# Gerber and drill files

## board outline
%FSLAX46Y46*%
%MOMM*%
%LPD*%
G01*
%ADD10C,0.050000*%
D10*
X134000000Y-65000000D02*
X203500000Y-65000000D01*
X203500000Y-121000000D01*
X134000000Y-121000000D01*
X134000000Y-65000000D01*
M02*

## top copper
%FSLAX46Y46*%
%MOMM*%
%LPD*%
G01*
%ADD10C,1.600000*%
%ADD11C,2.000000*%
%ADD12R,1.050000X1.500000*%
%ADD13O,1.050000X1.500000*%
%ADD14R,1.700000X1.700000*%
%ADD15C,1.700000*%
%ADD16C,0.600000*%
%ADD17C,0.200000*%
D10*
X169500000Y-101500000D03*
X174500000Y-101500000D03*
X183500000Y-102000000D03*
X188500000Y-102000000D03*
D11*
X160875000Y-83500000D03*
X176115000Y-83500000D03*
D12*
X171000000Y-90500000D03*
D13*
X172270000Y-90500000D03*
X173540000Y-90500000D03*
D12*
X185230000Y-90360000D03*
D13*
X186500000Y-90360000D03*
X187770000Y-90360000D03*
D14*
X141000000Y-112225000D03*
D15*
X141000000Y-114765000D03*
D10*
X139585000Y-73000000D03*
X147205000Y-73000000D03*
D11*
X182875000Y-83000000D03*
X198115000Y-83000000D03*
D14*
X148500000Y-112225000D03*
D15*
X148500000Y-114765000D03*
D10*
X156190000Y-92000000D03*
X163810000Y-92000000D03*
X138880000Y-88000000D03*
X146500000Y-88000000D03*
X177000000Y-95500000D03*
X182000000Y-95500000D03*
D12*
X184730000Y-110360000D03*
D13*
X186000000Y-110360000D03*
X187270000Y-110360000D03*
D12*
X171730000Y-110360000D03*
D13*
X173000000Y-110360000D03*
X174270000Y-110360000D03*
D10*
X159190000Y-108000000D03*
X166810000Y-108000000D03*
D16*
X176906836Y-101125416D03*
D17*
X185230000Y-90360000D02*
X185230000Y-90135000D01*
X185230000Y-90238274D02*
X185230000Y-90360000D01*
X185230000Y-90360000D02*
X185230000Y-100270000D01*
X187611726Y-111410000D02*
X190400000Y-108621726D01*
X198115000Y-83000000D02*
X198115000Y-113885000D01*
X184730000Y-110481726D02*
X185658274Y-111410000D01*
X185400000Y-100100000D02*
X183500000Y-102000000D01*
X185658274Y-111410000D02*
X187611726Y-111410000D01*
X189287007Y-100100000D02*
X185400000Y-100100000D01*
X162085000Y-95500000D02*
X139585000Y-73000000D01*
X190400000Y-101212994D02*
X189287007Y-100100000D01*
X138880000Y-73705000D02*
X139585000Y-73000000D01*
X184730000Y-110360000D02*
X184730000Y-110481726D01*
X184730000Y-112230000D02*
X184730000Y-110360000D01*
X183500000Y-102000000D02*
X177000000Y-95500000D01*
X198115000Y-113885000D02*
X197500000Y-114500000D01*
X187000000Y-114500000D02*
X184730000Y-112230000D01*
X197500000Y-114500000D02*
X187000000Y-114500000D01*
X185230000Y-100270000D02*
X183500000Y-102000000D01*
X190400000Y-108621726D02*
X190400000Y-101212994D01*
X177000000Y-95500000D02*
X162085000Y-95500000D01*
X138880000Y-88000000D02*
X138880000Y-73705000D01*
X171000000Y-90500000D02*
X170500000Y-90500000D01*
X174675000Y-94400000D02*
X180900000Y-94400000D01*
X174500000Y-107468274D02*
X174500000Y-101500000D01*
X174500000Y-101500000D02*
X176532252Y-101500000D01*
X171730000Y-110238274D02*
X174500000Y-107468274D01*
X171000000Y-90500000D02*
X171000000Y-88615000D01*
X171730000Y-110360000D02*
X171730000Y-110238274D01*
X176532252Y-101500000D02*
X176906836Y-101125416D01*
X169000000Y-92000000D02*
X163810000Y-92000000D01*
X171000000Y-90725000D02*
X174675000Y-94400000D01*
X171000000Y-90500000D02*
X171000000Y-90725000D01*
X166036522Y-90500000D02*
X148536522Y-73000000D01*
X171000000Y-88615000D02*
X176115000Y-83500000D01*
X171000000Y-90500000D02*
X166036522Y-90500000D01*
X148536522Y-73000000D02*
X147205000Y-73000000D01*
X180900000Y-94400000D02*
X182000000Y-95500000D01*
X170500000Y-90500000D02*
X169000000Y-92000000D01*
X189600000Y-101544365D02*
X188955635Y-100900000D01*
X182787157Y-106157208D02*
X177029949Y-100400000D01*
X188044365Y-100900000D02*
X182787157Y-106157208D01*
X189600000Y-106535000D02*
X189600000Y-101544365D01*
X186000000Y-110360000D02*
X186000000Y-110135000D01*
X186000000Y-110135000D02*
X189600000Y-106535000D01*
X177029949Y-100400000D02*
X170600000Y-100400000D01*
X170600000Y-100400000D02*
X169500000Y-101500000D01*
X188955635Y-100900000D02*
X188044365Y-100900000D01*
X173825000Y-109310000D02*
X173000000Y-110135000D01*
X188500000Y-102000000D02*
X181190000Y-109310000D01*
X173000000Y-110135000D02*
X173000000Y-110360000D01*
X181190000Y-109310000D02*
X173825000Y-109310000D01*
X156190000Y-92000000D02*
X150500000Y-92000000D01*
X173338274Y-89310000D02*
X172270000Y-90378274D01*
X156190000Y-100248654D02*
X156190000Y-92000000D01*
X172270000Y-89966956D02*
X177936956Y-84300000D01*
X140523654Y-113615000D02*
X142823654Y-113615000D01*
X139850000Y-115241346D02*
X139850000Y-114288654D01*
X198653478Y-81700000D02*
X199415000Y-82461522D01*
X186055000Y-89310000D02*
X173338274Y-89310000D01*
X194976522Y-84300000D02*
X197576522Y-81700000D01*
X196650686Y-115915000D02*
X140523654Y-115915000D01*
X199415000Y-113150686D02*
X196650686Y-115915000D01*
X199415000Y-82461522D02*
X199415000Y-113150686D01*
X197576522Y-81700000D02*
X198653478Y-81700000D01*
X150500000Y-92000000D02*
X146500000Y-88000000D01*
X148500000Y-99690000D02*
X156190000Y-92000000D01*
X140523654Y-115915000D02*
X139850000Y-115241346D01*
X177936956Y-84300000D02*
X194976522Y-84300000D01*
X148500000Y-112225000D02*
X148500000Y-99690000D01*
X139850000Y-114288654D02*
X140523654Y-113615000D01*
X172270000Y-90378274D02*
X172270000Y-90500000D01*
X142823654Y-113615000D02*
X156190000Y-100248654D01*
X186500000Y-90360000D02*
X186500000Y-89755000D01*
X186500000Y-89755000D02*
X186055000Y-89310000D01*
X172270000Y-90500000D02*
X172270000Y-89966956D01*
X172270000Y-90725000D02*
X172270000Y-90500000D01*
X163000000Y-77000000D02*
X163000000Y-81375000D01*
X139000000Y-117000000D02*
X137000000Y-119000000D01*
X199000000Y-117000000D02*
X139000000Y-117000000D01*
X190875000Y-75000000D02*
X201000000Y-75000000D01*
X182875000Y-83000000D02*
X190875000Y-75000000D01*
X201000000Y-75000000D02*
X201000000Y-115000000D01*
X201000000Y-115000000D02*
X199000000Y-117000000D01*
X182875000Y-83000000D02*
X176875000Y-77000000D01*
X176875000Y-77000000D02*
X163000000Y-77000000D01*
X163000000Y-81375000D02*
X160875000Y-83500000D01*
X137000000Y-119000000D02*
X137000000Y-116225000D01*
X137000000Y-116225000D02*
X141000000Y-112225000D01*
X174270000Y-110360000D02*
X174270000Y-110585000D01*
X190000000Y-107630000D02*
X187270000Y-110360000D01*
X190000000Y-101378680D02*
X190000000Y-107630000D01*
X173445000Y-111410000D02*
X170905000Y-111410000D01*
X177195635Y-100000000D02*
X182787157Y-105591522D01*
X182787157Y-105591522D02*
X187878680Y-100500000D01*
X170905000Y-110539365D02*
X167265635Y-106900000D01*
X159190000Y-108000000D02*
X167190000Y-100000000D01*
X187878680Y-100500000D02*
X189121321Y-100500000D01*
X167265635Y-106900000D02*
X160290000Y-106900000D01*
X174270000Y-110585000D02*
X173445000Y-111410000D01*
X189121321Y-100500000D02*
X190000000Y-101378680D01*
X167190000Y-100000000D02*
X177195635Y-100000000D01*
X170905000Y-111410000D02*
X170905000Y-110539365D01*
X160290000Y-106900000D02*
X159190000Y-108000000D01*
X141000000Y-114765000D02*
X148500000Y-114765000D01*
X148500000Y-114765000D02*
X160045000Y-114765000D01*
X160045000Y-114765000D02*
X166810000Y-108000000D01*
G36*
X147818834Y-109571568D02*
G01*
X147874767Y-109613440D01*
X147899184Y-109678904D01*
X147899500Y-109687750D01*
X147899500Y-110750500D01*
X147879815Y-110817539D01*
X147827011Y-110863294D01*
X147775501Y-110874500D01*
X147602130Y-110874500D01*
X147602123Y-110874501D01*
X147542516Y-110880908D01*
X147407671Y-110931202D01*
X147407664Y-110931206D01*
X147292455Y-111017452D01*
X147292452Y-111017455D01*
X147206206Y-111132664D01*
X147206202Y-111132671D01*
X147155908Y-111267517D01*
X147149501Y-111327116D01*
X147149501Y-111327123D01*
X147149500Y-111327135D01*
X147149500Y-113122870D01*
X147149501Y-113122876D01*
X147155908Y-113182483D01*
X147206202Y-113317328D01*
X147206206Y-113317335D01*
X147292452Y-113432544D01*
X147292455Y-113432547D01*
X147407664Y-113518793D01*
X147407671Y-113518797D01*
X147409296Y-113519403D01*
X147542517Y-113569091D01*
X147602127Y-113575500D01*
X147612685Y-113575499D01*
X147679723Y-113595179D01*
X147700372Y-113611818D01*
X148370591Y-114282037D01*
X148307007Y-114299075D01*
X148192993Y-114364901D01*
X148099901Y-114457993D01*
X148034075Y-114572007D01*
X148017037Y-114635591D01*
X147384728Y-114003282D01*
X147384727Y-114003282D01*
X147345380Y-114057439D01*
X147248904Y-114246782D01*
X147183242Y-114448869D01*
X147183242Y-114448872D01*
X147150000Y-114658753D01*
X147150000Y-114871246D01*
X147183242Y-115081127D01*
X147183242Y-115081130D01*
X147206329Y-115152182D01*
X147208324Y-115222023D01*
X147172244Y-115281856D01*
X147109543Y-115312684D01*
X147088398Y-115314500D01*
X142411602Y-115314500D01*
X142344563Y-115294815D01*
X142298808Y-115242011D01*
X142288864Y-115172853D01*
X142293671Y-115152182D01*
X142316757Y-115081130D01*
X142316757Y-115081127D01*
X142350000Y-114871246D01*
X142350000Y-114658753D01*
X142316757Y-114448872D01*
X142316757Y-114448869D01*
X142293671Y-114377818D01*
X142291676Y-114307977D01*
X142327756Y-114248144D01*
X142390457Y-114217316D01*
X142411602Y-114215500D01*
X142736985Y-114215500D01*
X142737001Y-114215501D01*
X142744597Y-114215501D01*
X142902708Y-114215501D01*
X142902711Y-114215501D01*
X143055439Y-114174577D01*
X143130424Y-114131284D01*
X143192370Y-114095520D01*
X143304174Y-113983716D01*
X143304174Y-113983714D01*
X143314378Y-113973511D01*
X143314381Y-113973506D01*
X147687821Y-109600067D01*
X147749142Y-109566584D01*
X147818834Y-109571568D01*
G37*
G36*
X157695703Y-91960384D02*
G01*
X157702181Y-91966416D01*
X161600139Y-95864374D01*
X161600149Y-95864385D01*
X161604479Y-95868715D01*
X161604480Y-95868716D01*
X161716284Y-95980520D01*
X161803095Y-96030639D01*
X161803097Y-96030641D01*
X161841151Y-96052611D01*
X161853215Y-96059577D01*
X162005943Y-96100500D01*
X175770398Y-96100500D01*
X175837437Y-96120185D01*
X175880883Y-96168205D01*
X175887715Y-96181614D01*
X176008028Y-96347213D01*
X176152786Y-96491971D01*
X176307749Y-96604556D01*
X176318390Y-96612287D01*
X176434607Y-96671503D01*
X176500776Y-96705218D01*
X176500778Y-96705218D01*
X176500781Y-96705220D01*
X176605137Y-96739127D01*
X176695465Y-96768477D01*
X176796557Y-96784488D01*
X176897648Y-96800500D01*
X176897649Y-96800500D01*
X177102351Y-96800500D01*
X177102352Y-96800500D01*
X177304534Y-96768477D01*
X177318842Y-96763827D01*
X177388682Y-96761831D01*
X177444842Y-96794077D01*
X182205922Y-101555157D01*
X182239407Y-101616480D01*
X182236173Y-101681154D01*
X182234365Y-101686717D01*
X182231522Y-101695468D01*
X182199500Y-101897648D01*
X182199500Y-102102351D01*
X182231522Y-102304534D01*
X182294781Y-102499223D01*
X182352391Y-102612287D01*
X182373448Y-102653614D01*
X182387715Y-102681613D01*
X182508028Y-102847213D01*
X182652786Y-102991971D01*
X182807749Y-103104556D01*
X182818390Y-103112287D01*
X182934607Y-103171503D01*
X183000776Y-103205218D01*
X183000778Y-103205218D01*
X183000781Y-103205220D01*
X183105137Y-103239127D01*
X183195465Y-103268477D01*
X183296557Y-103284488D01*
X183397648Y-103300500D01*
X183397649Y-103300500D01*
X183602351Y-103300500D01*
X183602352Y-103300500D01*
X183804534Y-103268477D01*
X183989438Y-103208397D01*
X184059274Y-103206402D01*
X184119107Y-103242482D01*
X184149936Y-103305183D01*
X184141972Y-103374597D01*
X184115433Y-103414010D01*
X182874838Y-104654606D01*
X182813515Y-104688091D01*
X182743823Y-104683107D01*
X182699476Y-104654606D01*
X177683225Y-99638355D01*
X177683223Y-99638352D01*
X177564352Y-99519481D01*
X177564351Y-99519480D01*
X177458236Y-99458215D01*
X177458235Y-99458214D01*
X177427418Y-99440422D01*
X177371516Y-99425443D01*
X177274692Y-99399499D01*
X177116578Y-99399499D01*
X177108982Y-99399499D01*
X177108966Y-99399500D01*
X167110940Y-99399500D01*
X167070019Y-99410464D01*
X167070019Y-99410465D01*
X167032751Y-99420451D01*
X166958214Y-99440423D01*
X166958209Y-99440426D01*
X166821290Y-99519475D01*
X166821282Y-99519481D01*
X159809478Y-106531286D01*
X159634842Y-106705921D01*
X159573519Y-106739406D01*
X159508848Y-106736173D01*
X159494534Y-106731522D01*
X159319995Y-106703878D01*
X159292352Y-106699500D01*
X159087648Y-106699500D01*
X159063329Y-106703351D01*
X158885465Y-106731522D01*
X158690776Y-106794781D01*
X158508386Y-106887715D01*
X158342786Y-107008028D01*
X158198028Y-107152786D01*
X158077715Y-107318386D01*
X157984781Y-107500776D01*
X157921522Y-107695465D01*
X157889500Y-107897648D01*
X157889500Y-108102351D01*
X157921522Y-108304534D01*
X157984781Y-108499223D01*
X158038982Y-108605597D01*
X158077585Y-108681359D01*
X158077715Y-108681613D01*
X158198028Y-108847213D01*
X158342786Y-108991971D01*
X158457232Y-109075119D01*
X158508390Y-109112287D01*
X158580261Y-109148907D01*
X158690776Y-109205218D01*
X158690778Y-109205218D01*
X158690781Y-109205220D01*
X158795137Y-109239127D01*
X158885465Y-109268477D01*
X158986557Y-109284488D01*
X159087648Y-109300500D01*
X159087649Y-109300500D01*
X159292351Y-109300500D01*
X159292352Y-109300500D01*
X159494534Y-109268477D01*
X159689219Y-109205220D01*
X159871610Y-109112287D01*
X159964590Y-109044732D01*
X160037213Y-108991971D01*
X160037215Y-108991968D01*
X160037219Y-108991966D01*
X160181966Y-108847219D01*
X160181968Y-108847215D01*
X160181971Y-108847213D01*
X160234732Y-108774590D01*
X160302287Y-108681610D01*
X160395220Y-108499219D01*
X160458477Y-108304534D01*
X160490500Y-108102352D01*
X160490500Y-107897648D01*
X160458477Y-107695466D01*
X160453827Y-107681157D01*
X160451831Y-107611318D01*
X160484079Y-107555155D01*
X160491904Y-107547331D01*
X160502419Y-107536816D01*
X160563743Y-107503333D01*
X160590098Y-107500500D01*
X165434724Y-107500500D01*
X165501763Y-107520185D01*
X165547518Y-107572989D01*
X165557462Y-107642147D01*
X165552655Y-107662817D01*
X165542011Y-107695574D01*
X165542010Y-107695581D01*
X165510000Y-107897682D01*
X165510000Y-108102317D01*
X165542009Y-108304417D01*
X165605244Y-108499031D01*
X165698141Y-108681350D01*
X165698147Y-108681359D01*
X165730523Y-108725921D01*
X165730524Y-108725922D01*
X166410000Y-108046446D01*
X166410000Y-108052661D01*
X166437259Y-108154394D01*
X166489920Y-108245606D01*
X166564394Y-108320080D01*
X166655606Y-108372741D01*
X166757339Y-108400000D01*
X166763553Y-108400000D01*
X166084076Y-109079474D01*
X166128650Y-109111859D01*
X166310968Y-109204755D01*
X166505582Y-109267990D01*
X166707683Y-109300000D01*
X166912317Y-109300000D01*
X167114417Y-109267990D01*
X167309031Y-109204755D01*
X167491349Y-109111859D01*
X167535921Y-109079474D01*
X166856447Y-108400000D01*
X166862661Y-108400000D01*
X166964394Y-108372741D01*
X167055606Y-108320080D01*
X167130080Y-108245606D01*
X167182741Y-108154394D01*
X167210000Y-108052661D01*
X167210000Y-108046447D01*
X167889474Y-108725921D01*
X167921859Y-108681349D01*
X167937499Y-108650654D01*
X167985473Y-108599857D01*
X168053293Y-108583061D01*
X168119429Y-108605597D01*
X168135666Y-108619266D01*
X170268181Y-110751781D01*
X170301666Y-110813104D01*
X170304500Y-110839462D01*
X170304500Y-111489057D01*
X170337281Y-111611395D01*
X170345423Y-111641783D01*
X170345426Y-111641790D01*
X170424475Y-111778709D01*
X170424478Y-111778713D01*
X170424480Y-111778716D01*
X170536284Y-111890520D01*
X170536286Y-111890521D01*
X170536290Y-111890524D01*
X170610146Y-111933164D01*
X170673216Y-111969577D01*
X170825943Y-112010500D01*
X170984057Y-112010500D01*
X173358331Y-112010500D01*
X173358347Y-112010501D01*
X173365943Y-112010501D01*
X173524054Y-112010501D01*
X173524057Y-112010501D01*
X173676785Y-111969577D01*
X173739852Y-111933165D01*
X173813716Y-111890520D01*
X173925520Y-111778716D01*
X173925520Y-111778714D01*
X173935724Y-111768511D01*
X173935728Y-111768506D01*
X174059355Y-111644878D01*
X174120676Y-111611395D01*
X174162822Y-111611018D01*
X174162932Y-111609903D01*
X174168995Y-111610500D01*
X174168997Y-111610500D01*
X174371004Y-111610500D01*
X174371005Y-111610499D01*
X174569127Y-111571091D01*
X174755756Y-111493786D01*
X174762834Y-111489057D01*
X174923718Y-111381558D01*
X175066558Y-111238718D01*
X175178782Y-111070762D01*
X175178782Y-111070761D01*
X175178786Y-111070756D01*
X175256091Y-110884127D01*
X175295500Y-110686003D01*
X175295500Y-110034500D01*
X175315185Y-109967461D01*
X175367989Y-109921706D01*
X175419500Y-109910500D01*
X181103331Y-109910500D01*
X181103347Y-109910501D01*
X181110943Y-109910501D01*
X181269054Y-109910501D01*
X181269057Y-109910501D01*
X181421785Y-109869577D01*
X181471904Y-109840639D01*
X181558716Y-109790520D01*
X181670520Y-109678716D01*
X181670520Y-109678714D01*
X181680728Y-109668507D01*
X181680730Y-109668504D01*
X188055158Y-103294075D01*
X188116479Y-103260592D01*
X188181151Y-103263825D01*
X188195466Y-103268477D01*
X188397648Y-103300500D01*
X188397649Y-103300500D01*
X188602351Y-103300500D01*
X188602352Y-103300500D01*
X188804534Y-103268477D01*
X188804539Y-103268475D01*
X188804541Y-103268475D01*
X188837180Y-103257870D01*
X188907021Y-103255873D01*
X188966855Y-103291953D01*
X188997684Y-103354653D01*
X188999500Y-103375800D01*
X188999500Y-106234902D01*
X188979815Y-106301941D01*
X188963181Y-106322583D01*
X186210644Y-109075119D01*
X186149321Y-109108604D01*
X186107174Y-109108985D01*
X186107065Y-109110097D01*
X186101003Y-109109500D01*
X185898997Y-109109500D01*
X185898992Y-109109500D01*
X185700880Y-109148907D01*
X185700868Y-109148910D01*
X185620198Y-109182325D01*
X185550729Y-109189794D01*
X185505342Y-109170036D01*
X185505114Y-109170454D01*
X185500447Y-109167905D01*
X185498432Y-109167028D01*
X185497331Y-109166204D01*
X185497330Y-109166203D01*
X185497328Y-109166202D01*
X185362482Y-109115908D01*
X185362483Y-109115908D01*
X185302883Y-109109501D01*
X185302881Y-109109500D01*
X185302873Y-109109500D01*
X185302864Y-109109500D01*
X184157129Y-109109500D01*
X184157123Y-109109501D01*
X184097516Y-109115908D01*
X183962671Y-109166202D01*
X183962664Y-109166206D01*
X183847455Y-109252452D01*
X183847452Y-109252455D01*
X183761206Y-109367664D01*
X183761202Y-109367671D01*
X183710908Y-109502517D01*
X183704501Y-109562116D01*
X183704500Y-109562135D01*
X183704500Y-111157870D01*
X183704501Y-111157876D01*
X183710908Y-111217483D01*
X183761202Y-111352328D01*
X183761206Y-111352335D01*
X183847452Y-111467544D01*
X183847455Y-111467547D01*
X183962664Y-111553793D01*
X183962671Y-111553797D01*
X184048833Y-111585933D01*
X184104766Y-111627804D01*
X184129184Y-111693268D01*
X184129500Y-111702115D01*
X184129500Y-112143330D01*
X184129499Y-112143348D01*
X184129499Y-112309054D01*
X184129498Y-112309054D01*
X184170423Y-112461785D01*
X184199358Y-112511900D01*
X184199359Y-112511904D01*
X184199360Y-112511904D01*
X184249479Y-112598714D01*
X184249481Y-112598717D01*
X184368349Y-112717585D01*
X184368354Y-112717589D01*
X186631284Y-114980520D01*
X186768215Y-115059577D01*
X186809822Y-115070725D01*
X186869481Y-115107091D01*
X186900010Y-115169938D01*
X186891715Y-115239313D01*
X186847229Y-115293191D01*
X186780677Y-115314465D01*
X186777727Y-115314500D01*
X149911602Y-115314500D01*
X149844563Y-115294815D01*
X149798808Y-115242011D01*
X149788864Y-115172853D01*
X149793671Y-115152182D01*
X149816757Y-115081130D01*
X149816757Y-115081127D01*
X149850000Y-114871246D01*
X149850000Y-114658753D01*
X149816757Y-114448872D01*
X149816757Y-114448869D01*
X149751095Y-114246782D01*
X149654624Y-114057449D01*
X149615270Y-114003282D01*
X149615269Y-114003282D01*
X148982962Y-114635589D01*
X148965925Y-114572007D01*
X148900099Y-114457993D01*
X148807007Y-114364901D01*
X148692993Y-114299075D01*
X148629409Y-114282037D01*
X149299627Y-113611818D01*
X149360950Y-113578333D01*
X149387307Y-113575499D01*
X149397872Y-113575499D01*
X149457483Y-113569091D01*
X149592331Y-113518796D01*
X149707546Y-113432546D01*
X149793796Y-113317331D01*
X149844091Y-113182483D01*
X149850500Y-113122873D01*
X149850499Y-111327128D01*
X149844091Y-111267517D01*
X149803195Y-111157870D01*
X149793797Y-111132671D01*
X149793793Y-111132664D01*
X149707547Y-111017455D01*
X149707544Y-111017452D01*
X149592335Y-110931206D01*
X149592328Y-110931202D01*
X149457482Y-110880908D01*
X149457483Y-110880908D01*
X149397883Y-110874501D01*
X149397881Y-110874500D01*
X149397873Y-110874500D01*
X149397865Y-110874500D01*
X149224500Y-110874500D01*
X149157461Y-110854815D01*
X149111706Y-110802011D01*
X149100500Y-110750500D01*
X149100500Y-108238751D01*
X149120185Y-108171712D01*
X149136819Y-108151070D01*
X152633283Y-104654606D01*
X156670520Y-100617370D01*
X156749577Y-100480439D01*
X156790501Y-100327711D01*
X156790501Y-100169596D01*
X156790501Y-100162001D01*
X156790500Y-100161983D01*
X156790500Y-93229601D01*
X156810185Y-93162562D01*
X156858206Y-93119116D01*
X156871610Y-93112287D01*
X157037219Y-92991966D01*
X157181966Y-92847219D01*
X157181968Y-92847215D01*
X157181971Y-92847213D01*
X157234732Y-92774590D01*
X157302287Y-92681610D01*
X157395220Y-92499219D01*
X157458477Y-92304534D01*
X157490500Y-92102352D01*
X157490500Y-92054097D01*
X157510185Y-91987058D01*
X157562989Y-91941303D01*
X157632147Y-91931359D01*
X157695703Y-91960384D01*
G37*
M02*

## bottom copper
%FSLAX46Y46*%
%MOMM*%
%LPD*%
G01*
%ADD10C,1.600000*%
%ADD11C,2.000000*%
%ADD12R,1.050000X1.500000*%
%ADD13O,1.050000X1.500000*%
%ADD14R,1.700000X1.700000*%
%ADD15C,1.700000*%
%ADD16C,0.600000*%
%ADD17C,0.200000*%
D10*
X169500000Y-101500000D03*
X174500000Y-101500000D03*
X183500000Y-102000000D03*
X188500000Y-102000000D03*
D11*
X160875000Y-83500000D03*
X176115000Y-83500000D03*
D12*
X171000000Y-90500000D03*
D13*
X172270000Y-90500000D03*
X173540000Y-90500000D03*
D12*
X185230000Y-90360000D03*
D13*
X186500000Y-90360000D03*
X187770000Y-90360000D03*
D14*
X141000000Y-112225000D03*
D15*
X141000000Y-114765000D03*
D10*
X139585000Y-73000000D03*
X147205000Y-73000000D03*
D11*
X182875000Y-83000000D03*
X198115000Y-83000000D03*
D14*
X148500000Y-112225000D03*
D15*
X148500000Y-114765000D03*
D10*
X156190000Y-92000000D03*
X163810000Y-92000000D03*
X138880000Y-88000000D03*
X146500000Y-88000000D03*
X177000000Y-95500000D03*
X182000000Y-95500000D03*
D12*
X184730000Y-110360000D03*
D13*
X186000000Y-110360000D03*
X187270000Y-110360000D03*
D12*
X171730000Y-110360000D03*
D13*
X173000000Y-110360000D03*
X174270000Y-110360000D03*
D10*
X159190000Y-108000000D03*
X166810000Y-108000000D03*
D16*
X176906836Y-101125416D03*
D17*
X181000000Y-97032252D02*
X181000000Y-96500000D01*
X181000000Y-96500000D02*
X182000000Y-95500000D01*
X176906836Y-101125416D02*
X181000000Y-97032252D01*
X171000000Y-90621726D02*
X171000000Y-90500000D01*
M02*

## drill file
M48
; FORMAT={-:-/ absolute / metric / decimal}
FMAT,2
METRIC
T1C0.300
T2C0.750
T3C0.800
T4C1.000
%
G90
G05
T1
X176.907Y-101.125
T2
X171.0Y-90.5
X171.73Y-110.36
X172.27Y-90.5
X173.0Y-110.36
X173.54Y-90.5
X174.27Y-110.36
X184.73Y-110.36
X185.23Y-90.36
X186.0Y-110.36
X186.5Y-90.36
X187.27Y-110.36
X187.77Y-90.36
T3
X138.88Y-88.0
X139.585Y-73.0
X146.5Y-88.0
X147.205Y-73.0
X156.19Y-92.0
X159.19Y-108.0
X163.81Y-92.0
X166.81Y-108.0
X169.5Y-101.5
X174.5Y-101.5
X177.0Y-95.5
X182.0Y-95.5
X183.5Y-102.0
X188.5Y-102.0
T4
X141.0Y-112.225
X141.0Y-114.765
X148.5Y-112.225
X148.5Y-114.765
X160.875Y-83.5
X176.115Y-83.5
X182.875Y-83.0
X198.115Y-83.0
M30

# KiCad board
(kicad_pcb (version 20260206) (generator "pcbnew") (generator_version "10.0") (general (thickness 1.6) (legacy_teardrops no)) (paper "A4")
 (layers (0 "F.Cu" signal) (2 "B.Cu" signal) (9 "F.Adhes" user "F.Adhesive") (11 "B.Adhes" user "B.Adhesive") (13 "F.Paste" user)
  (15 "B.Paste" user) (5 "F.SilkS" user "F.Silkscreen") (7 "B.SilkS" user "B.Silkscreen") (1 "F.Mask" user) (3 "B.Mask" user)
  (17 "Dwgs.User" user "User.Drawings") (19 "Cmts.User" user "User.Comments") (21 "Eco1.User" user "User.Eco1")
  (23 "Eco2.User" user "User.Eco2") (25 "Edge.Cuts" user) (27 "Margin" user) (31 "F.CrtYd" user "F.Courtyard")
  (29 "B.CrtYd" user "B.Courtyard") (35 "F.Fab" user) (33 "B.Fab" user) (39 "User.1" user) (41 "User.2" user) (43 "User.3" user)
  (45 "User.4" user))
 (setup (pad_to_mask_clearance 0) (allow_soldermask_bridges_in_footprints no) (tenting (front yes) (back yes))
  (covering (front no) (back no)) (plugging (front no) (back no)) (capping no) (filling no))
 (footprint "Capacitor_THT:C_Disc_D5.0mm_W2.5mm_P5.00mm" (layer "F.Cu") (at 169.5 101.5)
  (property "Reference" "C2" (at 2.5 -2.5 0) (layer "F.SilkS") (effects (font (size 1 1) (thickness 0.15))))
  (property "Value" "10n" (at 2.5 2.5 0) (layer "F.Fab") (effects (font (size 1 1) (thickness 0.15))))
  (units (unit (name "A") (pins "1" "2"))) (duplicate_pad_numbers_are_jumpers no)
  (pad "1" thru_hole circle (at 0 0) (size 1.6 1.6) (drill 0.8) (layers "*.Cu" "*.Mask") (remove_unused_layers no) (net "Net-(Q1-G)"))
  (pad "2" thru_hole circle (at 5 0) (size 1.6 1.6) (drill 0.8) (layers "*.Cu" "*.Mask") (remove_unused_layers no) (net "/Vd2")))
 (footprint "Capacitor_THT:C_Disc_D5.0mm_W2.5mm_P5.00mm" (layer "F.Cu") (at 183.5 102)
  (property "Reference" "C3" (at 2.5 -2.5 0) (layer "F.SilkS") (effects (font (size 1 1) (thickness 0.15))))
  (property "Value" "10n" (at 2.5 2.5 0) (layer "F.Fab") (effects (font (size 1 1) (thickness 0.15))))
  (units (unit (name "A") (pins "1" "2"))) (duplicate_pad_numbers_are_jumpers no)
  (pad "1" thru_hole circle (at 0 0) (size 1.6 1.6) (drill 0.8) (layers "*.Cu" "*.Mask") (remove_unused_layers no) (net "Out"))
  (pad "2" thru_hole circle (at 5 0) (size 1.6 1.6) (drill 0.8) (layers "*.Cu" "*.Mask") (remove_unused_layers no) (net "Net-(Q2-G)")))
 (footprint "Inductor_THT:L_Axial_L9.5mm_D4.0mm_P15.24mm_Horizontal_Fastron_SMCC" (layer "F.Cu") (at 160.875 83.5)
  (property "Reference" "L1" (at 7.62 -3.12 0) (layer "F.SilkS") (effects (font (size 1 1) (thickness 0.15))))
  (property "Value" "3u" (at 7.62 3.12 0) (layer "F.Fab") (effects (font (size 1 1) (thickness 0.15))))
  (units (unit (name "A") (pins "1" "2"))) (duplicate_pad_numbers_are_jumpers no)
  (pad "1" thru_hole circle (at 0 0) (size 2 2) (drill 1) (layers "*.Cu" "*.Mask") (remove_unused_layers no) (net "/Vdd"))
  (pad "2" thru_hole circle (at 15.24 0) (size 2 2) (drill 1) (layers "*.Cu" "*.Mask") (remove_unused_layers no) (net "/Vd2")))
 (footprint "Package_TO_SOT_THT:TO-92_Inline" (layer "F.Cu") (at 171 90.5)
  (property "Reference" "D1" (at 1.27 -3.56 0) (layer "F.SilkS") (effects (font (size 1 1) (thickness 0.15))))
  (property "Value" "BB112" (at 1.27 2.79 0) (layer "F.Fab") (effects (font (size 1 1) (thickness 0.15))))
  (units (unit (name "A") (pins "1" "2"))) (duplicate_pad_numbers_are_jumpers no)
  (pad "1" thru_hole rect (at 0 0) (size 1.05 1.5) (drill 0.75) (layers "*.Cu" "*.Mask") (remove_unused_layers no) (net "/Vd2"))
  (pad "2" thru_hole oval (at 1.27 0) (size 1.05 1.5) (drill 0.75) (layers "*.Cu" "*.Mask") (remove_unused_layers no) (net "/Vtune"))
  (pad "3" thru_hole oval (at 2.54 0) (size 1.05 1.5) (drill 0.75) (layers "*.Cu" "*.Mask") (remove_unused_layers no)))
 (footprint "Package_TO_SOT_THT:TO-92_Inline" (layer "F.Cu") (at 185.23 90.36)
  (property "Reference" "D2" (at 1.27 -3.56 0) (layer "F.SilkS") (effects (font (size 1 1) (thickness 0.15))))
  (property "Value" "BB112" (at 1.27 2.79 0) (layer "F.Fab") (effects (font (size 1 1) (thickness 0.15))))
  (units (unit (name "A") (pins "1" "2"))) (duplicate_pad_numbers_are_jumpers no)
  (pad "1" thru_hole rect (at 0 0) (size 1.05 1.5) (drill 0.75) (layers "*.Cu" "*.Mask") (remove_unused_layers no) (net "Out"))
  (pad "2" thru_hole oval (at 1.27 0) (size 1.05 1.5) (drill 0.75) (layers "*.Cu" "*.Mask") (remove_unused_layers no) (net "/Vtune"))
  (pad "3" thru_hole oval (at 2.54 0) (size 1.05 1.5) (drill 0.75) (layers "*.Cu" "*.Mask") (remove_unused_layers no)))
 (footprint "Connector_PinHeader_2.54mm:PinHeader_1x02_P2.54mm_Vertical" (layer "F.Cu") (at 141 112.225)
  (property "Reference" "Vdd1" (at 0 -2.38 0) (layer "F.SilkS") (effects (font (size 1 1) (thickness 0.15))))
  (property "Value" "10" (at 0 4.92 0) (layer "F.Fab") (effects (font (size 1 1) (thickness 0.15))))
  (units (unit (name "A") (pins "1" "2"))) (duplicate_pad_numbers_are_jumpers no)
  (pad "1" thru_hole rect (at 0 0) (size 1.7 1.7) (drill 1) (layers "*.Cu" "*.Mask") (remove_unused_layers no) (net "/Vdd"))
  (pad "2" thru_hole circle (at 0 2.54) (size 1.7 1.7) (drill 1) (layers "*.Cu" "*.Mask") (remove_unused_layers no) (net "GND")))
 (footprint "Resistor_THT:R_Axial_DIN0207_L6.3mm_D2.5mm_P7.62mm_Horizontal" (layer "F.Cu") (at 139.585 73)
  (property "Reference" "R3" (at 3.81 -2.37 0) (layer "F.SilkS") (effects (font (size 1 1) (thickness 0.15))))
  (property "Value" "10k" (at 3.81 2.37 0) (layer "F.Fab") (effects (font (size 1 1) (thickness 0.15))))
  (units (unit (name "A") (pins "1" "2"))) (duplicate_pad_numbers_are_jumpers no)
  (pad "1" thru_hole circle (at 0 0) (size 1.6 1.6) (drill 0.8) (layers "*.Cu" "*.Mask") (remove_unused_layers no) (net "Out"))
  (pad "2" thru_hole circle (at 7.62 0) (size 1.6 1.6) (drill 0.8) (layers "*.Cu" "*.Mask") (remove_unused_layers no) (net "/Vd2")))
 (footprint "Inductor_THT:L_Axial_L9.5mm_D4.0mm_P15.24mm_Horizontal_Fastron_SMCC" (layer "F.Cu") (at 182.875 83)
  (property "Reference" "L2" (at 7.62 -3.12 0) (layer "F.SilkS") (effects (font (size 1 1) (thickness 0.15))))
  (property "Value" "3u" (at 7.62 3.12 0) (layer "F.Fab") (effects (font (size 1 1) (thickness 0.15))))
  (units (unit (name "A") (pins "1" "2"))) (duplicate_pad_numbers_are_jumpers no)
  (pad "1" thru_hole circle (at 0 0) (size 2 2) (drill 1) (layers "*.Cu" "*.Mask") (remove_unused_layers no) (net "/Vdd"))
  (pad "2" thru_hole circle (at 15.24 0) (size 2 2) (drill 1) (layers "*.Cu" "*.Mask") (remove_unused_layers no) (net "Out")))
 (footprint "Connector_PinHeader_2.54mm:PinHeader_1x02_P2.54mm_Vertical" (layer "F.Cu") (at 148.5 112.225)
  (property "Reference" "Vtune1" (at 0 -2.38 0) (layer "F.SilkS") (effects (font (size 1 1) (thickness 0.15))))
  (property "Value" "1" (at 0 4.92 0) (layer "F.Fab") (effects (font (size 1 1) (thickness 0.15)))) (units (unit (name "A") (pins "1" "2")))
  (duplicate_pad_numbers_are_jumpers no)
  (pad "1" thru_hole rect (at 0 0) (size 1.7 1.7) (drill 1) (layers "*.Cu" "*.Mask") (remove_unused_layers no) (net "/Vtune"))
  (pad "2" thru_hole circle (at 0 2.54) (size 1.7 1.7) (drill 1) (layers "*.Cu" "*.Mask") (remove_unused_layers no) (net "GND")))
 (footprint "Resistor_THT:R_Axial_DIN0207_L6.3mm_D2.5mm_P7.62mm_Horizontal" (layer "F.Cu") (at 156.19 92)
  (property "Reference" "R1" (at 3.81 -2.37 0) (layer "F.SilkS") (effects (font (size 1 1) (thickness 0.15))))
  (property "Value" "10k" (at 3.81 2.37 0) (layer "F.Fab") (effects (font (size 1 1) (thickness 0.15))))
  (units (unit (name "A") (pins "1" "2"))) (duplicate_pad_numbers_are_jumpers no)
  (pad "1" thru_hole circle (at 0 0) (size 1.6 1.6) (drill 0.8) (layers "*.Cu" "*.Mask") (remove_unused_layers no) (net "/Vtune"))
  (pad "2" thru_hole circle (at 7.62 0) (size 1.6 1.6) (drill 0.8) (layers "*.Cu" "*.Mask") (remove_unused_layers no) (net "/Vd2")))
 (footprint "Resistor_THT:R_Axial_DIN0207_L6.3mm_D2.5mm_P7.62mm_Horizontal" (layer "F.Cu") (at 138.88 88)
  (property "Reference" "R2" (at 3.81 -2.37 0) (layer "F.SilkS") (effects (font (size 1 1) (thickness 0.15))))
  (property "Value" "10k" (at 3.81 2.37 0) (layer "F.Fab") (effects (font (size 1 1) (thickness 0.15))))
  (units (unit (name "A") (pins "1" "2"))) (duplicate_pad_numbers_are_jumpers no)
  (pad "1" thru_hole circle (at 0 0) (size 1.6 1.6) (drill 0.8) (layers "*.Cu" "*.Mask") (remove_unused_layers no) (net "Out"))
  (pad "2" thru_hole circle (at 7.62 0) (size 1.6 1.6) (drill 0.8) (layers "*.Cu" "*.Mask") (remove_unused_layers no) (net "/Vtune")))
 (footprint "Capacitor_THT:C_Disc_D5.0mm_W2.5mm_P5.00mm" (layer "F.Cu") (at 177 95.5)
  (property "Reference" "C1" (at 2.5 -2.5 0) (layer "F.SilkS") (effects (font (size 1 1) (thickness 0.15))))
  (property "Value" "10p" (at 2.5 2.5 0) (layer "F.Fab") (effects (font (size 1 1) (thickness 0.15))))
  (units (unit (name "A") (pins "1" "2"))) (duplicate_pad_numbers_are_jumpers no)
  (pad "1" thru_hole circle (at 0 0) (size 1.6 1.6) (drill 0.8) (layers "*.Cu" "*.Mask") (remove_unused_layers no) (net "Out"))
  (pad "2" thru_hole circle (at 5 0) (size 1.6 1.6) (drill 0.8) (layers "*.Cu" "*.Mask") (remove_unused_layers no) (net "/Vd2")))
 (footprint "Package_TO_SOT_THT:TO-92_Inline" (layer "F.Cu") (at 184.73 110.36)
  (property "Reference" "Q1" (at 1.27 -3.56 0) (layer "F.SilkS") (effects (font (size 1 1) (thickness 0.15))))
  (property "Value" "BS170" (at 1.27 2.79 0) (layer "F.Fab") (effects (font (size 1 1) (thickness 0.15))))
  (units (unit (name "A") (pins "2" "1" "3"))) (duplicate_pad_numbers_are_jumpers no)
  (pad "1" thru_hole rect (at 0 0) (size 1.05 1.5) (drill 0.75) (layers "*.Cu" "*.Mask") (remove_unused_layers no) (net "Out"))
  (pad "2" thru_hole oval (at 1.27 0) (size 1.05 1.5) (drill 0.75) (layers "*.Cu" "*.Mask") (remove_unused_layers no) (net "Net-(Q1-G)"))
  (pad "3" thru_hole oval (at 2.54 0) (size 1.05 1.5) (drill 0.75) (layers "*.Cu" "*.Mask") (remove_unused_layers no) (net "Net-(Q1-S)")))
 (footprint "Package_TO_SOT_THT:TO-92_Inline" (layer "F.Cu") (at 171.73 110.36)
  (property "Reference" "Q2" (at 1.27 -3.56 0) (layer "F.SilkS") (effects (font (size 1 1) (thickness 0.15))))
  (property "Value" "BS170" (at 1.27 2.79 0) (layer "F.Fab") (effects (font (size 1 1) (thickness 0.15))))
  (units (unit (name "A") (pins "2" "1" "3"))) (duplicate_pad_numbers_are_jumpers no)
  (pad "1" thru_hole rect (at 0 0) (size 1.05 1.5) (drill 0.75) (layers "*.Cu" "*.Mask") (remove_unused_layers no) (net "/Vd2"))
  (pad "2" thru_hole oval (at 1.27 0) (size 1.05 1.5) (drill 0.75) (layers "*.Cu" "*.Mask") (remove_unused_layers no) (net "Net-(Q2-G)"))
  (pad "3" thru_hole oval (at 2.54 0) (size 1.05 1.5) (drill 0.75) (layers "*.Cu" "*.Mask") (remove_unused_layers no) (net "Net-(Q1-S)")))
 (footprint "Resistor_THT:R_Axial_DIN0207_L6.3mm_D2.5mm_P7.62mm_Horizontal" (layer "F.Cu") (at 159.19 108)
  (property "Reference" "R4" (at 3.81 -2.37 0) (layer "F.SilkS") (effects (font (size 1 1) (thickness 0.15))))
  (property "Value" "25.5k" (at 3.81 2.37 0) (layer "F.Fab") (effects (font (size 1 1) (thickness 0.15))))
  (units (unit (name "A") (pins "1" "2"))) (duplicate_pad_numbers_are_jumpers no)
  (pad "1" thru_hole circle (at 0 0) (size 1.6 1.6) (drill 0.8) (layers "*.Cu" "*.Mask") (remove_unused_layers no) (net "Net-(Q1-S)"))
  (pad "2" thru_hole circle (at 7.62 0) (size 1.6 1.6) (drill 0.8) (layers "*.Cu" "*.Mask") (remove_unused_layers no) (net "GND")))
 (gr_rect (start 134 65) (end 203.5 121) (stroke (width 0.05) (type default)) (fill no) (layer "Edge.Cuts"))
 (segment (start 185.23 90.36) (end 185.23 90.135) (width 0.2) (layer "F.Cu") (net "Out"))
 (segment (start 185.23 90.238274) (end 185.23 90.36) (width 0.2) (layer "F.Cu") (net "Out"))
 (segment (start 185.23 90.36) (end 185.23 100.27) (width 0.2) (layer "F.Cu") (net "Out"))
 (segment (start 187.611726 111.41) (end 190.4 108.621726) (width 0.2) (layer "F.Cu") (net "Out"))
 (segment (start 198.115 83) (end 198.115 113.885) (width 0.2) (layer "F.Cu") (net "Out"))
 (segment (start 184.73 110.481726) (end 185.658274 111.41) (width 0.2) (layer "F.Cu") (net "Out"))
 (segment (start 185.4 100.1) (end 183.5 102) (width 0.2) (layer "F.Cu") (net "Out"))
 (segment (start 185.658274 111.41) (end 187.611726 111.41) (width 0.2) (layer "F.Cu") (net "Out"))
 (segment (start 189.287007 100.1) (end 185.4 100.1) (width 0.2) (layer "F.Cu") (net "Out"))
 (segment (start 162.085 95.5) (end 139.585 73) (width 0.2) (layer "F.Cu") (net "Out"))
 (segment (start 190.4 101.212994) (end 189.287007 100.1) (width 0.2) (layer "F.Cu") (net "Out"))
 (segment (start 138.88 73.705) (end 139.585 73) (width 0.2) (layer "F.Cu") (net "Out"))
 (segment (start 184.73 110.36) (end 184.73 110.481726) (width 0.2) (layer "F.Cu") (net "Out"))
 (segment (start 184.73 112.23) (end 184.73 110.36) (width 0.2) (layer "F.Cu") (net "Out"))
 (segment (start 183.5 102) (end 177 95.5) (width 0.2) (layer "F.Cu") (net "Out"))
 (segment (start 198.115 113.885) (end 197.5 114.5) (width 0.2) (layer "F.Cu") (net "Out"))
 (segment (start 187 114.5) (end 184.73 112.23) (width 0.2) (layer "F.Cu") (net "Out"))
 (segment (start 197.5 114.5) (end 187 114.5) (width 0.2) (layer "F.Cu") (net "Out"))
 (segment (start 185.23 100.27) (end 183.5 102) (width 0.2) (layer "F.Cu") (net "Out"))
 (segment (start 190.4 108.621726) (end 190.4 101.212994) (width 0.2) (layer "F.Cu") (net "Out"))
 (segment (start 177 95.5) (end 162.085 95.5) (width 0.2) (layer "F.Cu") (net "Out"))
 (segment (start 138.88 88) (end 138.88 73.705) (width 0.2) (layer "F.Cu") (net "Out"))
 (segment (start 171 90.5) (end 170.5 90.5) (width 0.2) (layer "F.Cu") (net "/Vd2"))
 (segment (start 174.675 94.4) (end 180.9 94.4) (width 0.2) (layer "F.Cu") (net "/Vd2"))
 (segment (start 174.5 107.468274) (end 174.5 101.5) (width 0.2) (layer "F.Cu") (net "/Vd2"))
 (segment (start 174.5 101.5) (end 176.532252 101.5) (width 0.2) (layer "F.Cu") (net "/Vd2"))
 (segment (start 171.73 110.238274) (end 174.5 107.468274) (width 0.2) (layer "F.Cu") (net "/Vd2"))
 (segment (start 171 90.5) (end 171 88.615) (width 0.2) (layer "F.Cu") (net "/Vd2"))
 (segment (start 171.73 110.36) (end 171.73 110.238274) (width 0.2) (layer "F.Cu") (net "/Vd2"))
 (segment (start 176.532252 101.5) (end 176.906836 101.125416) (width 0.2) (layer "F.Cu") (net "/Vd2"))
 (segment (start 169 92) (end 163.81 92) (width 0.2) (layer "F.Cu") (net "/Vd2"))
 (segment (start 171 90.725) (end 174.675 94.4) (width 0.2) (layer "F.Cu") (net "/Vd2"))
 (segment (start 171 90.5) (end 171 90.725) (width 0.2) (layer "F.Cu") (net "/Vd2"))
 (segment (start 166.036522 90.5) (end 148.536522 73) (width 0.2) (layer "F.Cu") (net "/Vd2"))
 (segment (start 171 88.615) (end 176.115 83.5) (width 0.2) (layer "F.Cu") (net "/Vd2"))
 (segment (start 171 90.5) (end 166.036522 90.5) (width 0.2) (layer "F.Cu") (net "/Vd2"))
 (segment (start 148.536522 73) (end 147.205 73) (width 0.2) (layer "F.Cu") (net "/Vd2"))
 (segment (start 180.9 94.4) (end 182 95.5) (width 0.2) (layer "F.Cu") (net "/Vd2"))
 (segment (start 170.5 90.5) (end 169 92) (width 0.2) (layer "F.Cu") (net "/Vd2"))
 (via (at 176.906836 101.125416) (size 0.6) (drill 0.3) (layers "F.Cu" "B.Cu") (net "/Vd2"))
 (segment (start 181 97.032252) (end 181 96.5) (width 0.2) (layer "B.Cu") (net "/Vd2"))
 (segment (start 181 96.5) (end 182 95.5) (width 0.2) (layer "B.Cu") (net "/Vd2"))
 (segment (start 176.906836 101.125416) (end 181 97.032252) (width 0.2) (layer "B.Cu") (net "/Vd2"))
 (segment (start 171 90.621726) (end 171 90.5) (width 0.2) (layer "B.Cu") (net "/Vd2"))
 (segment (start 189.6 101.544365) (end 188.955635 100.9) (width 0.2) (layer "F.Cu") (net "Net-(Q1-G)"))
 (segment (start 182.787157 106.157208) (end 177.029949 100.4) (width 0.2) (layer "F.Cu") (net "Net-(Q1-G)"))
 (segment (start 188.044365 100.9) (end 182.787157 106.157208) (width 0.2) (layer "F.Cu") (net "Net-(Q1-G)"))
 (segment (start 189.6 106.535) (end 189.6 101.544365) (width 0.2) (layer "F.Cu") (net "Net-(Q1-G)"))
 (segment (start 186 110.36) (end 186 110.135) (width 0.2) (layer "F.Cu") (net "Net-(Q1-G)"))
 (segment (start 186 110.135) (end 189.6 106.535) (width 0.2) (layer "F.Cu") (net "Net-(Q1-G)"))
 (segment (start 177.029949 100.4) (end 170.6 100.4) (width 0.2) (layer "F.Cu") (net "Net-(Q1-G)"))
 (segment (start 170.6 100.4) (end 169.5 101.5) (width 0.2) (layer "F.Cu") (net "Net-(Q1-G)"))
 (segment (start 188.955635 100.9) (end 188.044365 100.9) (width 0.2) (layer "F.Cu") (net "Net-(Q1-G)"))
 (segment (start 173.825 109.31) (end 173 110.135) (width 0.2) (layer "F.Cu") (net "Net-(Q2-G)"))
 (segment (start 188.5 102) (end 181.19 109.31) (width 0.2) (layer "F.Cu") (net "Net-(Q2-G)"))
 (segment (start 173 110.135) (end 173 110.36) (width 0.2) (layer "F.Cu") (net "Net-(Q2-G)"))
 (segment (start 181.19 109.31) (end 173.825 109.31) (width 0.2) (layer "F.Cu") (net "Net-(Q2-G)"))
 (segment (start 156.19 92) (end 150.5 92) (width 0.2) (layer "F.Cu") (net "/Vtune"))
 (segment (start 173.338274 89.31) (end 172.27 90.378274) (width 0.2) (layer "F.Cu") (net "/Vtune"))
 (segment (start 156.19 100.248654) (end 156.19 92) (width 0.2) (layer "F.Cu") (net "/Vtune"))
 (segment (start 172.27 89.966956) (end 177.936956 84.3) (width 0.2) (layer "F.Cu") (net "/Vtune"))
 (segment (start 140.523654 113.615) (end 142.823654 113.615) (width 0.2) (layer "F.Cu") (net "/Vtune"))
 (segment (start 139.85 115.241346) (end 139.85 114.288654) (width 0.2) (layer "F.Cu") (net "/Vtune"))
 (segment (start 198.653478 81.7) (end 199.415 82.461522) (width 0.2) (layer "F.Cu") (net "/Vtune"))
 (segment (start 186.055 89.31) (end 173.338274 89.31) (width 0.2) (layer "F.Cu") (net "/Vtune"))
 (segment (start 194.976522 84.3) (end 197.576522 81.7) (width 0.2) (layer "F.Cu") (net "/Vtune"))
 (segment (start 196.650686 115.915) (end 140.523654 115.915) (width 0.2) (layer "F.Cu") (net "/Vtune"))
 (segment (start 199.415 113.150686) (end 196.650686 115.915) (width 0.2) (layer "F.Cu") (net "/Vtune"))
 (segment (start 199.415 82.461522) (end 199.415 113.150686) (width 0.2) (layer "F.Cu") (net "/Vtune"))
 (segment (start 197.576522 81.7) (end 198.653478 81.7) (width 0.2) (layer "F.Cu") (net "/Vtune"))
 (segment (start 150.5 92) (end 146.5 88) (width 0.2) (layer "F.Cu") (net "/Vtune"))
 (segment (start 148.5 99.69) (end 156.19 92) (width 0.2) (layer "F.Cu") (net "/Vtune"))
 (segment (start 140.523654 115.915) (end 139.85 115.241346) (width 0.2) (layer "F.Cu") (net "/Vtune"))
 (segment (start 177.936956 84.3) (end 194.976522 84.3) (width 0.2) (layer "F.Cu") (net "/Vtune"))
 (segment (start 148.5 112.225) (end 148.5 99.69) (width 0.2) (layer "F.Cu") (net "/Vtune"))
 (segment (start 139.85 114.288654) (end 140.523654 113.615) (width 0.2) (layer "F.Cu") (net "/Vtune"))
 (segment (start 172.27 90.378274) (end 172.27 90.5) (width 0.2) (layer "F.Cu") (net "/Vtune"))
 (segment (start 142.823654 113.615) (end 156.19 100.248654) (width 0.2) (layer "F.Cu") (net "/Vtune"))
 (segment (start 186.5 90.36) (end 186.5 89.755) (width 0.2) (layer "F.Cu") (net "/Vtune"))
 (segment (start 186.5 89.755) (end 186.055 89.31) (width 0.2) (layer "F.Cu") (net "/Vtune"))
 (segment (start 172.27 90.5) (end 172.27 89.966956) (width 0.2) (layer "F.Cu") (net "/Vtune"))
 (segment (start 172.27 90.725) (end 172.27 90.5) (width 0.2) (layer "F.Cu") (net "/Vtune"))
 (segment (start 163 77) (end 163 81.375) (width 0.2) (layer "F.Cu") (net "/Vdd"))
 (segment (start 139 117) (end 137 119) (width 0.2) (layer "F.Cu") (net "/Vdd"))
 (segment (start 199 117) (end 139 117) (width 0.2) (layer "F.Cu") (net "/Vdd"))
 (segment (start 190.875 75) (end 201 75) (width 0.2) (layer "F.Cu") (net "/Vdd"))
 (segment (start 182.875 83) (end 190.875 75) (width 0.2) (layer "F.Cu") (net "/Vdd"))
 (segment (start 201 75) (end 201 115) (width 0.2) (layer "F.Cu") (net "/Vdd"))
 (segment (start 201 115) (end 199 117) (width 0.2) (layer "F.Cu") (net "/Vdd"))
 (segment (start 182.875 83) (end 176.875 77) (width 0.2) (layer "F.Cu") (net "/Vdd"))
 (segment (start 176.875 77) (end 163 77) (width 0.2) (layer "F.Cu") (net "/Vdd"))
 (segment (start 163 81.375) (end 160.875 83.5) (width 0.2) (layer "F.Cu") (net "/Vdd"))
 (segment (start 137 119) (end 137 116.225) (width 0.2) (layer "F.Cu") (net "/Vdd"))
 (segment (start 137 116.225) (end 141 112.225) (width 0.2) (layer "F.Cu") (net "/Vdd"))
 (segment (start 174.27 110.36) (end 174.27 110.585) (width 0.2) (layer "F.Cu") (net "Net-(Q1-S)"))
 (segment (start 190 107.63) (end 187.27 110.36) (width 0.2) (layer "F.Cu") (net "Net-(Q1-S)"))
 (segment (start 190 101.37868) (end 190 107.63) (width 0.2) (layer "F.Cu") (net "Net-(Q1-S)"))
 (segment (start 173.445 111.41) (end 170.905 111.41) (width 0.2) (layer "F.Cu") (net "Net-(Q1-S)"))
 (segment (start 177.195635 100) (end 182.787157 105.591522) (width 0.2) (layer "F.Cu") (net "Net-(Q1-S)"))
 (segment (start 182.787157 105.591522) (end 187.87868 100.5) (width 0.2) (layer "F.Cu") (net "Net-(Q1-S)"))
 (segment (start 170.905 110.539365) (end 167.265635 106.9) (width 0.2) (layer "F.Cu") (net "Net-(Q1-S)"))
 (segment (start 159.19 108) (end 167.19 100) (width 0.2) (layer "F.Cu") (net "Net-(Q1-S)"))
 (segment (start 187.87868 100.5) (end 189.121321 100.5) (width 0.2) (layer "F.Cu") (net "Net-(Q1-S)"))
 (segment (start 167.265635 106.9) (end 160.29 106.9) (width 0.2) (layer "F.Cu") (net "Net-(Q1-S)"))
 (segment (start 174.27 110.585) (end 173.445 111.41) (width 0.2) (layer "F.Cu") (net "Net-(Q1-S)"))
 (segment (start 189.121321 100.5) (end 190 101.37868) (width 0.2) (layer "F.Cu") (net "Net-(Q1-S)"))
 (segment (start 167.19 100) (end 177.195635 100) (width 0.2) (layer "F.Cu") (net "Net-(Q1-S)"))
 (segment (start 170.905 111.41) (end 170.905 110.539365) (width 0.2) (layer "F.Cu") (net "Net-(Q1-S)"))
 (segment (start 160.29 106.9) (end 159.19 108) (width 0.2) (layer "F.Cu") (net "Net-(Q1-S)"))
 (segment (start 141 114.765) (end 148.5 114.765) (width 0.2) (layer "F.Cu") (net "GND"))
 (segment (start 148.5 114.765) (end 160.045 114.765) (width 0.2) (layer "F.Cu") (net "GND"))
 (segment (start 160.045 114.765) (end 166.81 108) (width 0.2) (layer "F.Cu") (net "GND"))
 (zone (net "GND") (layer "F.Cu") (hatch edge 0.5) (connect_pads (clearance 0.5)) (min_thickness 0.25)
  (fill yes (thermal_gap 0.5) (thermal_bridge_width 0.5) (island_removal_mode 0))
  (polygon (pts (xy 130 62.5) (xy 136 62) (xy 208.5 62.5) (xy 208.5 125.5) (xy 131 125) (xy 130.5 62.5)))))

